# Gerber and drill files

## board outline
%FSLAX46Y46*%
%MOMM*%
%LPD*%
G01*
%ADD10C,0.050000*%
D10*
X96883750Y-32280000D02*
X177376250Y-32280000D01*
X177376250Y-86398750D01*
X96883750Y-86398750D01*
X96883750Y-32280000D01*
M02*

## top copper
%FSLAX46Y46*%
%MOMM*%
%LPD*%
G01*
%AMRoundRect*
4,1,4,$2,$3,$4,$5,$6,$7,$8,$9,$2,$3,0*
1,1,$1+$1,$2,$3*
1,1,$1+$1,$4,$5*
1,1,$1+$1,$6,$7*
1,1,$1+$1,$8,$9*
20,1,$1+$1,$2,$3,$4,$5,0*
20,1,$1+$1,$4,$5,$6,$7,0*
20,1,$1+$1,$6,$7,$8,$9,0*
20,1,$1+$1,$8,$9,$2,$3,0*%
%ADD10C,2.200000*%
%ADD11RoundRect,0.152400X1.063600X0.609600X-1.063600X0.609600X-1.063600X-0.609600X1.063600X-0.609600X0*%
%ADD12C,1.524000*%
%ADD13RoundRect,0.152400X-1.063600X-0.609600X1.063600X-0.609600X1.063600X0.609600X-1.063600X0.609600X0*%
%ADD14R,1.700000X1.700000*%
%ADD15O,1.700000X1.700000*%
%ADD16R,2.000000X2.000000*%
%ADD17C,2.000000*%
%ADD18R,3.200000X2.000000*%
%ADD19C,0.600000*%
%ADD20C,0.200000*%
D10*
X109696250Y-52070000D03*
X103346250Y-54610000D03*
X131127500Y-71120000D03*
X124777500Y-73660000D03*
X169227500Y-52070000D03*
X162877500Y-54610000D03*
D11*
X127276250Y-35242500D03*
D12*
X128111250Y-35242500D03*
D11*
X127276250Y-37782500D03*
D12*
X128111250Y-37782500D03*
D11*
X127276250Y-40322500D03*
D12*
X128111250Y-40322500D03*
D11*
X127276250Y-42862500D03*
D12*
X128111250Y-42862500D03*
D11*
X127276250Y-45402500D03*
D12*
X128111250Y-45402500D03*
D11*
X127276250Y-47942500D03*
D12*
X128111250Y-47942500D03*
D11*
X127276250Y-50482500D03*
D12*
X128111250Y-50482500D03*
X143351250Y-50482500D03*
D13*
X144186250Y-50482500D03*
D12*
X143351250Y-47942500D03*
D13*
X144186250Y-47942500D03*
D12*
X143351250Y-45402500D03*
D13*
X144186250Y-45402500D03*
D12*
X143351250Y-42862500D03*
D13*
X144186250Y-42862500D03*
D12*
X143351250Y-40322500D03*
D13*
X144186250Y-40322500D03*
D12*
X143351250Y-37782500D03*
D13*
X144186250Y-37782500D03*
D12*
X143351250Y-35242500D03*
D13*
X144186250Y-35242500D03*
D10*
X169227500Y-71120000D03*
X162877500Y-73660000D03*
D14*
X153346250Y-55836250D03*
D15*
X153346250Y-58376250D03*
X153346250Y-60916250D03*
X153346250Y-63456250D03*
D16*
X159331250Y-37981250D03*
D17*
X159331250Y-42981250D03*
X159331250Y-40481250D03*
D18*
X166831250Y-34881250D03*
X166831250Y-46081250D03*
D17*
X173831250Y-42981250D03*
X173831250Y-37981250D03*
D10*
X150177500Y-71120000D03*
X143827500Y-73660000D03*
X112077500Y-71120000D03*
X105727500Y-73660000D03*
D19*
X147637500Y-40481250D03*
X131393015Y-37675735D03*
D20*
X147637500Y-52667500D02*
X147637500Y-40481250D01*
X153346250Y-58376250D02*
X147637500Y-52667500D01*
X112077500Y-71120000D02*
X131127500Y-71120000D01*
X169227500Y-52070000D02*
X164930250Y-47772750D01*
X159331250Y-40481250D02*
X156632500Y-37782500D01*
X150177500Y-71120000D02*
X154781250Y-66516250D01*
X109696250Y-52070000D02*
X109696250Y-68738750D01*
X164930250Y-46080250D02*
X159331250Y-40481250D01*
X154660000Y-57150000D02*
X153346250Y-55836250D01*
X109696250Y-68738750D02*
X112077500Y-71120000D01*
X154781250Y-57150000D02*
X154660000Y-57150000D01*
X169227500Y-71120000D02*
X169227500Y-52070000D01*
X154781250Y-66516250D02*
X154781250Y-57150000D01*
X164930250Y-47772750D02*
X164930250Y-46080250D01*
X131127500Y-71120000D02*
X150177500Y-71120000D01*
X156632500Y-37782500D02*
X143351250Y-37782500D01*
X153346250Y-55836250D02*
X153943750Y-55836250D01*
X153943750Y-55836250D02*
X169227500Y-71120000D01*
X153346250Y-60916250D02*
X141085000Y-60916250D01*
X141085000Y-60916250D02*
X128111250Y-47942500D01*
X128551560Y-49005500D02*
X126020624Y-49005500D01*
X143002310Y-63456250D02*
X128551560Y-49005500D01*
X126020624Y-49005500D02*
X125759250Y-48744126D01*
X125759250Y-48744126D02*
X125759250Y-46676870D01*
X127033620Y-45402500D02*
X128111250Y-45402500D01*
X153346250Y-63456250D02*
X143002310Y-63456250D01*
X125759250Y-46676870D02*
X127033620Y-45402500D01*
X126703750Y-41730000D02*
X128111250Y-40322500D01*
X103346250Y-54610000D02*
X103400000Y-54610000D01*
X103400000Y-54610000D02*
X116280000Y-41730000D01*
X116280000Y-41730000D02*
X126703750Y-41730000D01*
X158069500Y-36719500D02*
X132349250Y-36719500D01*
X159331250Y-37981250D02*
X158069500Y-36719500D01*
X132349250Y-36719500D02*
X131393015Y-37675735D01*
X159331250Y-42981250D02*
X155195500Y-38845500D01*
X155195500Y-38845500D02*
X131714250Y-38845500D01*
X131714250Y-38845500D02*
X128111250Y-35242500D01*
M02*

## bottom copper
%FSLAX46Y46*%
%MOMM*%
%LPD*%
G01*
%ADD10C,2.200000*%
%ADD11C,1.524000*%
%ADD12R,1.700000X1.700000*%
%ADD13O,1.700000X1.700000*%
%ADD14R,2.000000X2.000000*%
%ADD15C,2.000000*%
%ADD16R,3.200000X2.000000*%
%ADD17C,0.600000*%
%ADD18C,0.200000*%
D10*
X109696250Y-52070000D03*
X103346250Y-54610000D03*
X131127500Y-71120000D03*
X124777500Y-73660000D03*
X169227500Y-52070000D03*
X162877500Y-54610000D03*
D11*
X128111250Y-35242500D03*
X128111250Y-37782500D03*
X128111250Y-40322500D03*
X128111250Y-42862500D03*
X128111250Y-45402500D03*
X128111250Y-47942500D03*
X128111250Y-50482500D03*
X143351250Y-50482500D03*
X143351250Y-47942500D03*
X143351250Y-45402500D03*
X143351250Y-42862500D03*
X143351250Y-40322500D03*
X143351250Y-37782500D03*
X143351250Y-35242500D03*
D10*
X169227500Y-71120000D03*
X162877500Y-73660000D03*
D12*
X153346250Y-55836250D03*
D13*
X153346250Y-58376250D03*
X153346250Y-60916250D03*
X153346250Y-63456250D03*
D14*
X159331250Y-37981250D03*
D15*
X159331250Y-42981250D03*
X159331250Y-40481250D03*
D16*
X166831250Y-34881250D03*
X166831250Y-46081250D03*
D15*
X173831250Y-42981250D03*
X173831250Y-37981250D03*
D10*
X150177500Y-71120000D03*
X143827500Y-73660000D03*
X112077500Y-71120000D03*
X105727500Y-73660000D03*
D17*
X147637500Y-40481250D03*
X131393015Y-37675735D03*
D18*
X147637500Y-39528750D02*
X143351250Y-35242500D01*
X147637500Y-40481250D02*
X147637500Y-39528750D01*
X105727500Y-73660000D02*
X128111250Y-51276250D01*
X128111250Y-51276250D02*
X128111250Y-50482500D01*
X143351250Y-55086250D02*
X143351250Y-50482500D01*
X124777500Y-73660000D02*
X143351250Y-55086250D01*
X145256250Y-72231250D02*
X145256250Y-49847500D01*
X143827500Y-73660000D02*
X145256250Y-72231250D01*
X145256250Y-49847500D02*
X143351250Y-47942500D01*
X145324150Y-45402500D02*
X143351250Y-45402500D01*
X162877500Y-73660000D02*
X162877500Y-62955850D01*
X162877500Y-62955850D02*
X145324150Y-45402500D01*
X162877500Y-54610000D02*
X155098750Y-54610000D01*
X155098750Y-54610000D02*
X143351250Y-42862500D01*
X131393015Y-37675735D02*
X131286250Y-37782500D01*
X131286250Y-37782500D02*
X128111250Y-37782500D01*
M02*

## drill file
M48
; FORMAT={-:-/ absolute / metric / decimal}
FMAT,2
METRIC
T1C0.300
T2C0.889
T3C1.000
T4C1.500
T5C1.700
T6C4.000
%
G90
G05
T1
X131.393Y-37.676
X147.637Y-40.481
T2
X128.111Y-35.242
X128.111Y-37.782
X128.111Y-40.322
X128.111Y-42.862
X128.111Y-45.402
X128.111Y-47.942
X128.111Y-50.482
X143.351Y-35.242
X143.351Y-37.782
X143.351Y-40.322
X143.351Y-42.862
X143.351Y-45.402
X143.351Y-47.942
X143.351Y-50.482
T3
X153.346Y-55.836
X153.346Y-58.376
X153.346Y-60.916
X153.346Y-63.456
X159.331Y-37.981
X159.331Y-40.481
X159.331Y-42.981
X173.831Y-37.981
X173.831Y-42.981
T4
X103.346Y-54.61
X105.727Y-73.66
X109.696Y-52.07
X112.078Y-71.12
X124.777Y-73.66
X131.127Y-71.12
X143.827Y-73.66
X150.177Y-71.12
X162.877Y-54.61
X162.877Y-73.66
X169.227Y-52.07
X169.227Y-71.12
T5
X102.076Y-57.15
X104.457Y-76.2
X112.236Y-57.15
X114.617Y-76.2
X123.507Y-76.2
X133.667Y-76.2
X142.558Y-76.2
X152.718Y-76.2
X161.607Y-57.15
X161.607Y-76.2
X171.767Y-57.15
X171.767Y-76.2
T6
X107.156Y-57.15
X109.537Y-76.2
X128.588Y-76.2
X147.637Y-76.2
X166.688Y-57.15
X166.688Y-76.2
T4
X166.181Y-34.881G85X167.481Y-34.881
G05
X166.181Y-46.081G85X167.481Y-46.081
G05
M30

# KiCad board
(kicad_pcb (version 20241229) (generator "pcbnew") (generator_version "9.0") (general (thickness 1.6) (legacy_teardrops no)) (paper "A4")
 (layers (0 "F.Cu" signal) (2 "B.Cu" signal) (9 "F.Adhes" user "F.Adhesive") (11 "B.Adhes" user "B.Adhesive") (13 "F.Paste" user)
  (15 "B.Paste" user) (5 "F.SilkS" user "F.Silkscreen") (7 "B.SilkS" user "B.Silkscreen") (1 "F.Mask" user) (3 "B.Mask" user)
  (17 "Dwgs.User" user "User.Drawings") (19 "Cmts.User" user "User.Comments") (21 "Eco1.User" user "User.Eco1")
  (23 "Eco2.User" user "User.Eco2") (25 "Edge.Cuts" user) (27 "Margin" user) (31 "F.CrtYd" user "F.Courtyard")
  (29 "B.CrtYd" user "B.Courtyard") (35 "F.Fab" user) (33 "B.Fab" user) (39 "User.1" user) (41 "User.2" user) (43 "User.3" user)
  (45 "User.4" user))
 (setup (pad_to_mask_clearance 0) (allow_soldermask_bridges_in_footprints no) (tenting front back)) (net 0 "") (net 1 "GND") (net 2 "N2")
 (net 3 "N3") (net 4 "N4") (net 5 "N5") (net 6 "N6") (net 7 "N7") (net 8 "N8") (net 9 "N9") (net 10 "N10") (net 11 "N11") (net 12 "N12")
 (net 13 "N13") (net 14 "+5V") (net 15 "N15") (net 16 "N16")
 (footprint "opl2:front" (layer "F.Cu") (at 104.86 38.67)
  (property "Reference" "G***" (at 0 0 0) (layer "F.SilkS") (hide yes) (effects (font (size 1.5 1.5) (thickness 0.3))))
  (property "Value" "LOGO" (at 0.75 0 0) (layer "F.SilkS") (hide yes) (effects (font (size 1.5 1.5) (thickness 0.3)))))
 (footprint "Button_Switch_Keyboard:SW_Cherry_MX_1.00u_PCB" (layer "F.Cu") (at 109.69625 52.07)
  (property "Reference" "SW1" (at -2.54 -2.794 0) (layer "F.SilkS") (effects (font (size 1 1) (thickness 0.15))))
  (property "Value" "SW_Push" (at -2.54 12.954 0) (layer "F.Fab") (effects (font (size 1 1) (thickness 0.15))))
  (pad "" np_thru_hole circle (at -7.62 5.08) (size 1.7 1.7) (drill 1.7) (layers "*.Cu" "*.Mask"))
  (pad "" np_thru_hole circle (at -2.54 5.08) (size 4 4) (drill 4) (layers "*.Cu" "*.Mask"))
  (pad "" np_thru_hole circle (at 2.54 5.08) (size 1.7 1.7) (drill 1.7) (layers "*.Cu" "*.Mask"))
  (pad "1" thru_hole circle (at 0 0) (size 2.2 2.2) (drill 1.5) (layers "*.Cu" "*.Mask") (remove_unused_layers no) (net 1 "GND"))
  (pad "2" thru_hole circle (at -6.35 2.54) (size 2.2 2.2) (drill 1.5) (layers "*.Cu" "*.Mask") (remove_unused_layers no) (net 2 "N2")))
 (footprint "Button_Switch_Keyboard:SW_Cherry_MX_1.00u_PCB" (layer "F.Cu") (at 131.1275 71.12)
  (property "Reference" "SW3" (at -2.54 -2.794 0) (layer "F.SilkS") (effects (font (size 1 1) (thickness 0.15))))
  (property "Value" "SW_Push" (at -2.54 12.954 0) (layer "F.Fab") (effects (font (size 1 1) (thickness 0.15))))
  (pad "" np_thru_hole circle (at -7.62 5.08) (size 1.7 1.7) (drill 1.7) (layers "*.Cu" "*.Mask"))
  (pad "" np_thru_hole circle (at -2.54 5.08) (size 4 4) (drill 4) (layers "*.Cu" "*.Mask"))
  (pad "" np_thru_hole circle (at 2.54 5.08) (size 1.7 1.7) (drill 1.7) (layers "*.Cu" "*.Mask"))
  (pad "1" thru_hole circle (at 0 0) (size 2.2 2.2) (drill 1.5) (layers "*.Cu" "*.Mask") (remove_unused_layers no) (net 1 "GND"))
  (pad "2" thru_hole circle (at -6.35 2.54) (size 2.2 2.2) (drill 1.5) (layers "*.Cu" "*.Mask") (remove_unused_layers no) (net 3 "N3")))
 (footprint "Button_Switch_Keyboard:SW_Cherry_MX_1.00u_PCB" (layer "F.Cu") (at 169.2275 52.07)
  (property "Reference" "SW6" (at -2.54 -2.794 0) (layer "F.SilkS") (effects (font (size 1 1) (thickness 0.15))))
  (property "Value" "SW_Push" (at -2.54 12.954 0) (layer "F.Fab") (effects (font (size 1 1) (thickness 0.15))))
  (pad "" np_thru_hole circle (at -7.62 5.08) (size 1.7 1.7) (drill 1.7) (layers "*.Cu" "*.Mask"))
  (pad "" np_thru_hole circle (at -2.54 5.08) (size 4 4) (drill 4) (layers "*.Cu" "*.Mask"))
  (pad "" np_thru_hole circle (at 2.54 5.08) (size 1.7 1.7) (drill 1.7) (layers "*.Cu" "*.Mask"))
  (pad "1" thru_hole circle (at 0 0) (size 2.2 2.2) (drill 1.5) (layers "*.Cu" "*.Mask") (remove_unused_layers no) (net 1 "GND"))
  (pad "2" thru_hole circle (at -6.35 2.54) (size 2.2 2.2) (drill 1.5) (layers "*.Cu" "*.Mask") (remove_unused_layers no) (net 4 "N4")))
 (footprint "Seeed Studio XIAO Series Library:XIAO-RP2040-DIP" (layer "F.Cu") (at 135.73125 42.8625)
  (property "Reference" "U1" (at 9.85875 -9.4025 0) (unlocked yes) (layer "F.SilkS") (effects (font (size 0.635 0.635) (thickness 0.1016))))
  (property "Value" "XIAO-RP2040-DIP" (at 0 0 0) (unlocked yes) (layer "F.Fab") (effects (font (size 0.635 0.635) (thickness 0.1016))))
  (pad "1" smd roundrect (at -8.455 -7.62 180) (size 2.432 1.524) (layers "F.Cu" "F.Mask") (roundrect_rratio 0.1) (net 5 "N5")
   (thermal_bridge_angle 45))
  (pad "1" thru_hole circle (at -7.62 -7.62 180) (size 1.524 1.524) (drill 0.889) (layers "*.Cu" "*.Mask") (remove_unused_layers no)
   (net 5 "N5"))
  (pad "2" smd roundrect (at -8.455 -5.08 180) (size 2.432 1.524) (layers "F.Cu" "F.Mask") (roundrect_rratio 0.1) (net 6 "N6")
   (thermal_bridge_angle 45))
  (pad "2" thru_hole circle (at -7.62 -5.08 180) (size 1.524 1.524) (drill 0.889) (layers "*.Cu" "*.Mask") (remove_unused_layers no)
   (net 6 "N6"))
  (pad "3" smd roundrect (at -8.455 -2.54 180) (size 2.432 1.524) (layers "F.Cu" "F.Mask") (roundrect_rratio 0.1) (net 2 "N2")
   (thermal_bridge_angle 45))
  (pad "3" thru_hole circle (at -7.62 -2.54 180) (size 1.524 1.524) (drill 0.889) (layers "*.Cu" "*.Mask") (remove_unused_layers no)
   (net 2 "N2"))
  (pad "4" smd roundrect (at -8.455 0 180) (size 2.432 1.524) (layers "F.Cu" "F.Mask") (roundrect_rratio 0.1) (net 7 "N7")
   (thermal_bridge_angle 45))
  (pad "4" thru_hole circle (at -7.62 0 180) (size 1.524 1.524) (drill 0.889) (layers "*.Cu" "*.Mask") (remove_unused_layers no)
   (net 7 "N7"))
  (pad "5" smd roundrect (at -8.455 2.54 180) (size 2.432 1.524) (layers "F.Cu" "F.Mask") (roundrect_rratio 0.1) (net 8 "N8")
   (thermal_bridge_angle 45))
  (pad "5" thru_hole circle (at -7.62 2.54 180) (size 1.524 1.524) (drill 0.889) (layers "*.Cu" "*.Mask") (remove_unused_layers no)
   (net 8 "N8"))
  (pad "6" smd roundrect (at -8.455 5.08 180) (size 2.432 1.524) (layers "F.Cu" "F.Mask") (roundrect_rratio 0.1) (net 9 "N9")
   (thermal_bridge_angle 45))
  (pad "6" thru_hole circle (at -7.62 5.08 180) (size 1.524 1.524) (drill 0.889) (layers "*.Cu" "*.Mask") (remove_unused_layers no)
   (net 9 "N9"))
  (pad "7" smd roundrect (at -8.455 7.62 180) (size 2.432 1.524) (layers "F.Cu" "F.Mask") (roundrect_rratio 0.1) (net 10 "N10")
   (thermal_bridge_angle 45))
  (pad "7" thru_hole circle (at -7.62 7.62 180) (size 1.524 1.524) (drill 0.889) (layers "*.Cu" "*.Mask") (remove_unused_layers no)
   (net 10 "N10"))
  (pad "8" thru_hole circle (at 7.62 7.62) (size 1.524 1.524) (drill 0.889) (layers "*.Cu" "*.Mask") (remove_unused_layers no) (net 3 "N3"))
  (pad "8" smd roundrect (at 8.455 7.62) (size 2.432 1.524) (layers "F.Cu" "F.Mask") (roundrect_rratio 0.1) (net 3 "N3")
   (thermal_bridge_angle 45))
  (pad "9" thru_hole circle (at 7.62 5.08) (size 1.524 1.524) (drill 0.889) (layers "*.Cu" "*.Mask") (remove_unused_layers no)
   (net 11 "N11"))
  (pad "9" smd roundrect (at 8.455 5.08) (size 2.432 1.524) (layers "F.Cu" "F.Mask") (roundrect_rratio 0.1) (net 11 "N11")
   (thermal_bridge_angle 45))
  (pad "10" thru_hole circle (at 7.62 2.54) (size 1.524 1.524) (drill 0.889) (layers "*.Cu" "*.Mask") (remove_unused_layers no)
   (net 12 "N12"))
  (pad "10" smd roundrect (at 8.455 2.54) (size 2.432 1.524) (layers "F.Cu" "F.Mask") (roundrect_rratio 0.1) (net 12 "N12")
   (thermal_bridge_angle 45))
  (pad "11" thru_hole circle (at 7.62 0) (size 1.524 1.524) (drill 0.889) (layers "*.Cu" "*.Mask") (remove_unused_layers no) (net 4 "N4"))
  (pad "11" smd roundrect (at 8.455 0) (size 2.432 1.524) (layers "F.Cu" "F.Mask") (roundrect_rratio 0.1) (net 4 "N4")
   (thermal_bridge_angle 45))
  (pad "12" thru_hole circle (at 7.62 -2.54) (size 1.524 1.524) (drill 0.889) (layers "*.Cu" "*.Mask") (remove_unused_layers no)
   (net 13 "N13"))
  (pad "12" smd roundrect (at 8.455 -2.54) (size 2.432 1.524) (layers "F.Cu" "F.Mask") (roundrect_rratio 0.1) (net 13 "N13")
   (thermal_bridge_angle 45))
  (pad "13" thru_hole circle (at 7.62 -5.08) (size 1.524 1.524) (drill 0.889) (layers "*.Cu" "*.Mask") (remove_unused_layers no)
   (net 1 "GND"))
  (pad "13" smd roundrect (at 8.455 -5.08) (size 2.432 1.524) (layers "F.Cu" "F.Mask") (roundrect_rratio 0.1) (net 1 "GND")
   (thermal_bridge_angle 45))
  (pad "14" thru_hole circle (at 7.62 -7.62) (size 1.524 1.524) (drill 0.889) (layers "*.Cu" "*.Mask") (remove_unused_layers no)
   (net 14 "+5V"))
  (pad "14" smd roundrect (at 8.455 -7.62) (size 2.432 1.524) (layers "F.Cu" "F.Mask") (roundrect_rratio 0.1) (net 14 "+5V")
   (thermal_bridge_angle 45)))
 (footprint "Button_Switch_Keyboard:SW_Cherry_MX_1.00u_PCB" (layer "F.Cu") (at 169.2275 71.12)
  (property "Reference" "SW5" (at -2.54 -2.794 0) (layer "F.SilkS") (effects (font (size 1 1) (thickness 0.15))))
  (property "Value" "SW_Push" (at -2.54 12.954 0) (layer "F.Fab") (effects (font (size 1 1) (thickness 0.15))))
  (pad "" np_thru_hole circle (at -7.62 5.08) (size 1.7 1.7) (drill 1.7) (layers "*.Cu" "*.Mask"))
  (pad "" np_thru_hole circle (at -2.54 5.08) (size 4 4) (drill 4) (layers "*.Cu" "*.Mask"))
  (pad "" np_thru_hole circle (at 2.54 5.08) (size 1.7 1.7) (drill 1.7) (layers "*.Cu" "*.Mask"))
  (pad "1" thru_hole circle (at 0 0) (size 2.2 2.2) (drill 1.5) (layers "*.Cu" "*.Mask") (remove_unused_layers no) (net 1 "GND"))
  (pad "2" thru_hole circle (at -6.35 2.54) (size 2.2 2.2) (drill 1.5) (layers "*.Cu" "*.Mask") (remove_unused_layers no) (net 12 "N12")))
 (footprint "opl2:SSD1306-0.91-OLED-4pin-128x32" (layer "F.Cu") (at 116.84625 53.64625)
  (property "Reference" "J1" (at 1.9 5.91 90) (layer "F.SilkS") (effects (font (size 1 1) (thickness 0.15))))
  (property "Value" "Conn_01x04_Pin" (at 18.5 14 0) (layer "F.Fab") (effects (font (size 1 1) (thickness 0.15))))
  (pad "1" thru_hole rect (at 36.5 2.19) (size 1.7 1.7) (drill 1) (layers "*.Cu" "*.Mask") (remove_unused_layers no) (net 1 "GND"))
  (pad "2" thru_hole oval (at 36.5 4.73) (size 1.7 1.7) (drill 1) (layers "*.Cu" "*.Mask") (remove_unused_layers no) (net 14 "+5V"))
  (pad "3" thru_hole oval (at 36.5 7.27) (size 1.7 1.7) (drill 1) (layers "*.Cu" "*.Mask") (remove_unused_layers no) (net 9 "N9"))
  (pad "4" thru_hole oval (at 36.5 9.81) (size 1.7 1.7) (drill 1) (layers "*.Cu" "*.Mask") (remove_unused_layers no) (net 8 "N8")))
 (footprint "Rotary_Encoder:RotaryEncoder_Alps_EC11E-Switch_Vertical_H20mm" (layer "F.Cu") (at 159.33125 37.98125)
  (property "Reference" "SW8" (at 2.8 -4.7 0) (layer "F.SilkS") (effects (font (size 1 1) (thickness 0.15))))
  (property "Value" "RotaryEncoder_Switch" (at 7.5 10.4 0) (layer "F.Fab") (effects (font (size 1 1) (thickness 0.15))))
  (pad "A" thru_hole rect (at 0 0) (size 2 2) (drill 1) (layers "*.Cu" "*.Mask") (remove_unused_layers no) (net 6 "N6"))
  (pad "B" thru_hole circle (at 0 5) (size 2 2) (drill 1) (layers "*.Cu" "*.Mask") (remove_unused_layers no) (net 5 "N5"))
  (pad "C" thru_hole circle (at 0 2.5) (size 2 2) (drill 1) (layers "*.Cu" "*.Mask") (remove_unused_layers no) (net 1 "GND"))
  (pad "MP" thru_hole rect (at 7.5 -3.1) (size 3.2 2) (drill oval 2.8 1.5) (layers "*.Cu" "*.Mask") (remove_unused_layers no))
  (pad "MP" thru_hole rect (at 7.5 8.1) (size 3.2 2) (drill oval 2.8 1.5) (layers "*.Cu" "*.Mask") (remove_unused_layers no))
  (pad "S1" thru_hole circle (at 14.5 5) (size 2 2) (drill 1) (layers "*.Cu" "*.Mask") (remove_unused_layers no) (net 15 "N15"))
  (pad "S2" thru_hole circle (at 14.5 0) (size 2 2) (drill 1) (layers "*.Cu" "*.Mask") (remove_unused_layers no) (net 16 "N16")))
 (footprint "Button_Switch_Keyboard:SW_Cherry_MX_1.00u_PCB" (layer "F.Cu") (at 150.1775 71.12)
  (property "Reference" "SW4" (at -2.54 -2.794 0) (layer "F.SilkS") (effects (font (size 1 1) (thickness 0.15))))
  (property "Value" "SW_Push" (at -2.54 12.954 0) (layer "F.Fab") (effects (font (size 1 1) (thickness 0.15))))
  (pad "" np_thru_hole circle (at -7.62 5.08) (size 1.7 1.7) (drill 1.7) (layers "*.Cu" "*.Mask"))
  (pad "" np_thru_hole circle (at -2.54 5.08) (size 4 4) (drill 4) (layers "*.Cu" "*.Mask"))
  (pad "" np_thru_hole circle (at 2.54 5.08) (size 1.7 1.7) (drill 1.7) (layers "*.Cu" "*.Mask"))
  (pad "1" thru_hole circle (at 0 0) (size 2.2 2.2) (drill 1.5) (layers "*.Cu" "*.Mask") (remove_unused_layers no) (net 1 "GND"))
  (pad "2" thru_hole circle (at -6.35 2.54) (size 2.2 2.2) (drill 1.5) (layers "*.Cu" "*.Mask") (remove_unused_layers no) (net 11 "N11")))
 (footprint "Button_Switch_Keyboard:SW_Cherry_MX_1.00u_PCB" (layer "F.Cu") (at 112.0775 71.12)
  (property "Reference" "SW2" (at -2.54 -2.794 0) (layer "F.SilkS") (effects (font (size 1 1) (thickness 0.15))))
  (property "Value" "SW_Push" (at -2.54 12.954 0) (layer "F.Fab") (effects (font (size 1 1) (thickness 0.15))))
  (pad "" np_thru_hole circle (at -7.62 5.08) (size 1.7 1.7) (drill 1.7) (layers "*.Cu" "*.Mask"))
  (pad "" np_thru_hole circle (at -2.54 5.08) (size 4 4) (drill 4) (layers "*.Cu" "*.Mask"))
  (pad "" np_thru_hole circle (at 2.54 5.08) (size 1.7 1.7) (drill 1.7) (layers "*.Cu" "*.Mask"))
  (pad "1" thru_hole circle (at 0 0) (size 2.2 2.2) (drill 1.5) (layers "*.Cu" "*.Mask") (remove_unused_layers no) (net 1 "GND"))
  (pad "2" thru_hole circle (at -6.35 2.54) (size 2.2 2.2) (drill 1.5) (layers "*.Cu" "*.Mask") (remove_unused_layers no) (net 10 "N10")))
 (gr_rect (start 96.88375 32.28) (end 177.37625 86.39875) (stroke (width 0.05) (type default)) (fill no) (layer "Edge.Cuts"))
 (segment (start 147.6375 52.6675) (end 147.6375 40.48125) (width 0.2) (layer "F.Cu") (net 14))
 (segment (start 153.34625 58.37625) (end 147.6375 52.6675) (width 0.2) (layer "F.Cu") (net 14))
 (via (at 147.6375 40.48125) (size 0.6) (drill 0.3) (layers "F.Cu" "B.Cu") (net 14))
 (segment (start 147.6375 39.52875) (end 143.35125 35.2425) (width 0.2) (layer "B.Cu") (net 14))
 (segment (start 147.6375 40.48125) (end 147.6375 39.52875) (width 0.2) (layer "B.Cu") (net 14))
 (segment (start 112.0775 71.12) (end 131.1275 71.12) (width 0.2) (layer "F.Cu") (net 1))
 (segment (start 169.2275 52.07) (end 164.93025 47.77275) (width 0.2) (layer "F.Cu") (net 1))
 (segment (start 159.33125 40.48125) (end 156.6325 37.7825) (width 0.2) (layer "F.Cu") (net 1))
 (segment (start 150.1775 71.12) (end 154.78125 66.51625) (width 0.2) (layer "F.Cu") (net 1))
 (segment (start 109.69625 52.07) (end 109.69625 68.73875) (width 0.2) (layer "F.Cu") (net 1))
 (segment (start 164.93025 46.08025) (end 159.33125 40.48125) (width 0.2) (layer "F.Cu") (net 1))
 (segment (start 154.66 57.15) (end 153.34625 55.83625) (width 0.2) (layer "F.Cu") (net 1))
 (segment (start 109.69625 68.73875) (end 112.0775 71.12) (width 0.2) (layer "F.Cu") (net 1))
 (segment (start 154.78125 57.15) (end 154.66 57.15) (width 0.2) (layer "F.Cu") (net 1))
 (segment (start 169.2275 71.12) (end 169.2275 52.07) (width 0.2) (layer "F.Cu") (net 1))
 (segment (start 154.78125 66.51625) (end 154.78125 57.15) (width 0.2) (layer "F.Cu") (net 1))
 (segment (start 164.93025 47.77275) (end 164.93025 46.08025) (width 0.2) (layer "F.Cu") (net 1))
 (segment (start 131.1275 71.12) (end 150.1775 71.12) (width 0.2) (layer "F.Cu") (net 1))
 (segment (start 156.6325 37.7825) (end 143.35125 37.7825) (width 0.2) (layer "F.Cu") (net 1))
 (segment (start 153.34625 55.83625) (end 153.94375 55.83625) (width 0.2) (layer "F.Cu") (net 1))
 (segment (start 153.94375 55.83625) (end 169.2275 71.12) (width 0.2) (layer "F.Cu") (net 1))
 (segment (start 153.34625 60.91625) (end 141.085 60.91625) (width 0.2) (layer "F.Cu") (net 9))
 (segment (start 141.085 60.91625) (end 128.11125 47.9425) (width 0.2) (layer "F.Cu") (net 9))
 (segment (start 128.55156 49.0055) (end 126.020624 49.0055) (width 0.2) (layer "F.Cu") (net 8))
 (segment (start 143.00231 63.45625) (end 128.55156 49.0055) (width 0.2) (layer "F.Cu") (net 8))
 (segment (start 126.020624 49.0055) (end 125.75925 48.744126) (width 0.2) (layer "F.Cu") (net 8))
 (segment (start 125.75925 48.744126) (end 125.75925 46.67687) (width 0.2) (layer "F.Cu") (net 8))
 (segment (start 127.03362 45.4025) (end 128.11125 45.4025) (width 0.2) (layer "F.Cu") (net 8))
 (segment (start 153.34625 63.45625) (end 143.00231 63.45625) (width 0.2) (layer "F.Cu") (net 8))
 (segment (start 125.75925 46.67687) (end 127.03362 45.4025) (width 0.2) (layer "F.Cu") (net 8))
 (segment (start 126.70375 41.73) (end 128.11125 40.3225) (width 0.2) (layer "F.Cu") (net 2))
 (segment (start 103.34625 54.61) (end 103.4 54.61) (width 0.2) (layer "F.Cu") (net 2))
 (segment (start 103.4 54.61) (end 116.28 41.73) (width 0.2) (layer "F.Cu") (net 2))
 (segment (start 116.28 41.73) (end 126.70375 41.73) (width 0.2) (layer "F.Cu") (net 2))
 (segment (start 105.7275 73.66) (end 128.11125 51.27625) (width 0.2) (layer "B.Cu") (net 10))
 (segment (start 128.11125 51.27625) (end 128.11125 50.4825) (width 0.2) (layer "B.Cu") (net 10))
 (segment (start 143.35125 55.08625) (end 143.35125 50.4825) (width 0.2) (layer "B.Cu") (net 3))
 (segment (start 124.7775 73.66) (end 143.35125 55.08625) (width 0.2) (layer "B.Cu") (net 3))
 (segment (start 145.25625 72.23125) (end 145.25625 49.8475) (width 0.2) (layer "B.Cu") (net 11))
 (segment (start 143.8275 73.66) (end 145.25625 72.23125) (width 0.2) (layer "B.Cu") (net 11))
 (segment (start 145.25625 49.8475) (end 143.35125 47.9425) (width 0.2) (layer "B.Cu") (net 11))
 (segment (start 145.32415 45.4025) (end 143.35125 45.4025) (width 0.2) (layer "B.Cu") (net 12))
 (segment (start 162.8775 73.66) (end 162.8775 62.95585) (width 0.2) (layer "B.Cu") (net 12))
 (segment (start 162.8775 62.95585) (end 145.32415 45.4025) (width 0.2) (layer "B.Cu") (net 12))
 (segment (start 162.8775 54.61) (end 155.09875 54.61) (width 0.2) (layer "B.Cu") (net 4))
 (segment (start 155.09875 54.61) (end 143.35125 42.8625) (width 0.2) (layer "B.Cu") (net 4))
 (segment (start 158.0695 36.7195) (end 132.34925 36.7195) (width 0.2) (layer "F.Cu") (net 6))
 (segment (start 159.33125 37.98125) (end 158.0695 36.7195) (width 0.2) (layer "F.Cu") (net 6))
 (segment (start 132.34925 36.7195) (end 131.393015 37.675735) (width 0.2) (layer "F.Cu") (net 6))
 (via (at 131.393015 37.675735) (size 0.6) (drill 0.3) (layers "F.Cu" "B.Cu") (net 6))
 (segment (start 131.393015 37.675735) (end 131.28625 37.7825) (width 0.2) (layer "B.Cu") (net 6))
 (segment (start 131.28625 37.7825) (end 128.11125 37.7825) (width 0.2) (layer "B.Cu") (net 6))
 (segment (start 159.33125 42.98125) (end 155.1955 38.8455) (width 0.2) (layer "F.Cu") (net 5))
 (segment (start 155.1955 38.8455) (end 131.71425 38.8455) (width 0.2) (layer "F.Cu") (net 5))
 (segment (start 131.71425 38.8455) (end 128.11125 35.2425) (width 0.2) (layer "F.Cu") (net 5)))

